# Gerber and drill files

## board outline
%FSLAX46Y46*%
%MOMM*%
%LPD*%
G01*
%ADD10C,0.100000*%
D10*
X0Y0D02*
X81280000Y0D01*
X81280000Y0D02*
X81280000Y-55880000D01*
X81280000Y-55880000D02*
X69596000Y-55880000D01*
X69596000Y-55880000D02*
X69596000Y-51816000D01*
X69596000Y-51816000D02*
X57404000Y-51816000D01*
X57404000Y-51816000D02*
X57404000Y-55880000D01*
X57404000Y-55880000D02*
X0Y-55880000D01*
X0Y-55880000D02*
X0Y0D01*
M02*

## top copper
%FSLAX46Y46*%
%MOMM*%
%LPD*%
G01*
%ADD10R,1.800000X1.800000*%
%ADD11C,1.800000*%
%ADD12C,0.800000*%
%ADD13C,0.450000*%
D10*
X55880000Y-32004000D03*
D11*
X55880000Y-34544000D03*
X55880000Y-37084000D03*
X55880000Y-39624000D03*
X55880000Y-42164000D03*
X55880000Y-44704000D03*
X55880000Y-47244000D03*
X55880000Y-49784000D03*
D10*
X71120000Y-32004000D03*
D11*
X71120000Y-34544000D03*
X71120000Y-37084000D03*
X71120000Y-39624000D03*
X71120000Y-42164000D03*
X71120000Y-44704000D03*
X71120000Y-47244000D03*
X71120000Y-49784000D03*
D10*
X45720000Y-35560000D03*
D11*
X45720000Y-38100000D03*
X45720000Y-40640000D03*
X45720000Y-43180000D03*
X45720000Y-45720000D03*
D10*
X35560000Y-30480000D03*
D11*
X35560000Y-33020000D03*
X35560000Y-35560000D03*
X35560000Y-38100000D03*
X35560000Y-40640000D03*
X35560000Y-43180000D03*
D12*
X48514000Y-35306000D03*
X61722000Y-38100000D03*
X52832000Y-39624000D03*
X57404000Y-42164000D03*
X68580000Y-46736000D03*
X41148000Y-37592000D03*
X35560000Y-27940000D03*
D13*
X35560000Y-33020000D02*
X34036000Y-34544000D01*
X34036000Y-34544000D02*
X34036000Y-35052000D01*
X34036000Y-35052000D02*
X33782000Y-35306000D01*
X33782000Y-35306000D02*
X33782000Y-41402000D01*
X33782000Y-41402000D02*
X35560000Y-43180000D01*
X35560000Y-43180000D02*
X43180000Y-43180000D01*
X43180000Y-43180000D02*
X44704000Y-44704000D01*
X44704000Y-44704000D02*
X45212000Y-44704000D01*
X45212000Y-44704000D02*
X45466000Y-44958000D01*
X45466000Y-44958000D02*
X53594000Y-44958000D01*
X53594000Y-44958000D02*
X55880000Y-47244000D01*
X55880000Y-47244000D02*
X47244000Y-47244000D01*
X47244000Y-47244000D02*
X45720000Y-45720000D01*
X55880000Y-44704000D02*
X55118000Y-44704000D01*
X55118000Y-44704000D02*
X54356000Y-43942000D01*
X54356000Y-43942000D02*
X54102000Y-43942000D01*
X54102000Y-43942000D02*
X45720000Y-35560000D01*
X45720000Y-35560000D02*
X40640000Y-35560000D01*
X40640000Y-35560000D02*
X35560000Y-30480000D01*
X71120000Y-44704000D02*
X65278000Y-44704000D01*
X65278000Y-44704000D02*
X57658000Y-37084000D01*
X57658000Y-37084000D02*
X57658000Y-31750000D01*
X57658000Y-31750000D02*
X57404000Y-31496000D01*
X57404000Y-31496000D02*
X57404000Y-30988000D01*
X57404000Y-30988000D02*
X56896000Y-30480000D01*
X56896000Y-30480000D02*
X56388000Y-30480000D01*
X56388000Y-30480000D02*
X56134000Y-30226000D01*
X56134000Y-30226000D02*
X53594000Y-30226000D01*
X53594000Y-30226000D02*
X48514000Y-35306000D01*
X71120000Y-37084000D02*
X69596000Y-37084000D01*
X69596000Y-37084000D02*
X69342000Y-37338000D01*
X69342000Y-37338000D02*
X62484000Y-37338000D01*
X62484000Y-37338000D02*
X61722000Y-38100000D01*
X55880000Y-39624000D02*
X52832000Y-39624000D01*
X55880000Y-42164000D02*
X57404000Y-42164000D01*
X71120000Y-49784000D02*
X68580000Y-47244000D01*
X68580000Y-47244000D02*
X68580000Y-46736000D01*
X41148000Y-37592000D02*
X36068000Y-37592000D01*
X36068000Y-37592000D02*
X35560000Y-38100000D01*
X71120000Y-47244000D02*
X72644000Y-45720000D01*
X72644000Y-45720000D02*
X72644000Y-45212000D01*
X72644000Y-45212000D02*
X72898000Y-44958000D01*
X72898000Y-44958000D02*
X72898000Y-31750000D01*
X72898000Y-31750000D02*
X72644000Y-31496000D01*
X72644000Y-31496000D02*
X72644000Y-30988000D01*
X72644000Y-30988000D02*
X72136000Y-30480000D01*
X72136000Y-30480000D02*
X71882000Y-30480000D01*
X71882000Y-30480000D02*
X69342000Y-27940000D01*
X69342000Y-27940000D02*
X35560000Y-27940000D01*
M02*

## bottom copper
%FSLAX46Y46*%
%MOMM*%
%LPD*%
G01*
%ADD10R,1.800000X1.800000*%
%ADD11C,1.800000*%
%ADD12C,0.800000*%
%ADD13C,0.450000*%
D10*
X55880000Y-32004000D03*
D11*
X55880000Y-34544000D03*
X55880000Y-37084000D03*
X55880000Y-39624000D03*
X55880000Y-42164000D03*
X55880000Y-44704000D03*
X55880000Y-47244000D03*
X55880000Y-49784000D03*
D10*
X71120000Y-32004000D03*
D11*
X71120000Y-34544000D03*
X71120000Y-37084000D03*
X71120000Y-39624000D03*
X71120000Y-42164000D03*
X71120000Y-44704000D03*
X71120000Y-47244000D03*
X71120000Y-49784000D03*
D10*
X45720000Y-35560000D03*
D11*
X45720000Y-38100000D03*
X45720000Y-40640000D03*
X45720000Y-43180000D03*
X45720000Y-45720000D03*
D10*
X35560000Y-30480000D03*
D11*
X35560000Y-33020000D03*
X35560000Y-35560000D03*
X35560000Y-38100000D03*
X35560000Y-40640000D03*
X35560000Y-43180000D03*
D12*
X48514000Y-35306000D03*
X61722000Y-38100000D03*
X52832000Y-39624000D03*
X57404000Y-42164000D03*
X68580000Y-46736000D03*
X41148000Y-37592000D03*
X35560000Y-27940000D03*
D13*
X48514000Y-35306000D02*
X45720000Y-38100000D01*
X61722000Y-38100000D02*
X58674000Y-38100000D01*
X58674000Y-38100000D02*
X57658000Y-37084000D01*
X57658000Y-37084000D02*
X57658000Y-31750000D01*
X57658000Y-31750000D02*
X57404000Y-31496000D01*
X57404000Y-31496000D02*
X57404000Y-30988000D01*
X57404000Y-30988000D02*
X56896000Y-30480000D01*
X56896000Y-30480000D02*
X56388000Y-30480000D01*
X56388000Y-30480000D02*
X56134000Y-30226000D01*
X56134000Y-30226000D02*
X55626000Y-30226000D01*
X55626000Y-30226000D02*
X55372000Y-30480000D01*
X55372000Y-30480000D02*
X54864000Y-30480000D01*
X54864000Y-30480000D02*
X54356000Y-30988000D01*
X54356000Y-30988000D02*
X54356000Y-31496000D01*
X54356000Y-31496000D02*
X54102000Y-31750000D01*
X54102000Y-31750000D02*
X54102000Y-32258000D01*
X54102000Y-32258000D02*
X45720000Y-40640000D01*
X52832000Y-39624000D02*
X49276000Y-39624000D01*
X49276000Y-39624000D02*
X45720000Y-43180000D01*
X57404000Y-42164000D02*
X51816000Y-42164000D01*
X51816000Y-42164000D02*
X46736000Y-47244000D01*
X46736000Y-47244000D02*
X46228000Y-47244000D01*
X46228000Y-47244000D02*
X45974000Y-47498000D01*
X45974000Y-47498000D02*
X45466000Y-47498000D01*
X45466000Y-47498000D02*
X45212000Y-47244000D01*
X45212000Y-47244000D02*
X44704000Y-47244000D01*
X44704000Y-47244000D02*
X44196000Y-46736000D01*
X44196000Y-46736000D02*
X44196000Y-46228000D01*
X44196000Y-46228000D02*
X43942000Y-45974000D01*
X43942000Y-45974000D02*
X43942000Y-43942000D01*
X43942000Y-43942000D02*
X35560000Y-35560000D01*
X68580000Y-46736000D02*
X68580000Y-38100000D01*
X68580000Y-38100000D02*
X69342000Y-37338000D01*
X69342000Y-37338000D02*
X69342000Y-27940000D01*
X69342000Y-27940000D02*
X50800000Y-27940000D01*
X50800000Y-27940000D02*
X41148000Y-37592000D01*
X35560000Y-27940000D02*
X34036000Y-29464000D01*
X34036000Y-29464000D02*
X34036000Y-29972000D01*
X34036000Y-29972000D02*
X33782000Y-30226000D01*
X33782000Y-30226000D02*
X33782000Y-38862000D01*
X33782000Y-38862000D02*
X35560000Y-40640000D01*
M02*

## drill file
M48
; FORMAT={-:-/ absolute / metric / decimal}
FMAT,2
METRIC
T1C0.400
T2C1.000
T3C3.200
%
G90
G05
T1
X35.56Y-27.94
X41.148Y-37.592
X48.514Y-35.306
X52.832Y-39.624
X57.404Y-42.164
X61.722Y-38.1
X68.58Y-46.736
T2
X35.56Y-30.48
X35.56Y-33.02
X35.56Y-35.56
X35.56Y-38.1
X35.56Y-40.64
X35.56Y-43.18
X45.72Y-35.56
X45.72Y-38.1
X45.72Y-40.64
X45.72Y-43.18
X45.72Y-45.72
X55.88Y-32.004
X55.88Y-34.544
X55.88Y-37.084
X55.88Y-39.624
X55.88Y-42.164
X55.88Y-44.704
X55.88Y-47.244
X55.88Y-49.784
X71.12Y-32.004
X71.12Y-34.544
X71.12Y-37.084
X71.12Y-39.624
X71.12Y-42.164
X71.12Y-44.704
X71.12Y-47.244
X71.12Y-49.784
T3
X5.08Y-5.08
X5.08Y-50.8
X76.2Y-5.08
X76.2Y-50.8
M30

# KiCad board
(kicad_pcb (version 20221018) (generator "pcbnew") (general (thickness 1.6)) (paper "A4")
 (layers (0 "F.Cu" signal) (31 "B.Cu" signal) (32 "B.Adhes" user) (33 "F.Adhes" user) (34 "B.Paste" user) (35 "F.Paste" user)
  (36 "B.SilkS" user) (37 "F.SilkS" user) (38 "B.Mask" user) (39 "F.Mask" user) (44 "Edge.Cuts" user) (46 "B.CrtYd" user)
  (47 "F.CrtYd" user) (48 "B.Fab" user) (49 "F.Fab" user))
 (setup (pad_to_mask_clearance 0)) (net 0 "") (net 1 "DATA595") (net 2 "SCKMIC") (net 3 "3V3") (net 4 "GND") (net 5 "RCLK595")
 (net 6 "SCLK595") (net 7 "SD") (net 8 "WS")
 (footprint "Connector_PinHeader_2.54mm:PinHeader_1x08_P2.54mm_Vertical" (layer "F.Cu") (at 55.8800 32.0040)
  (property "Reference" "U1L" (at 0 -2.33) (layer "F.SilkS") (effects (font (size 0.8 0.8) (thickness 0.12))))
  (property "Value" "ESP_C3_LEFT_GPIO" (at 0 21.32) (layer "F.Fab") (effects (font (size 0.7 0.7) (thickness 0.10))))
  (pad "1" thru_hole rect (at 0 0.0000) (size 1.8 1.8) (drill 1.0) (layers "*.Cu" "*.Mask") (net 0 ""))
  (pad "2" thru_hole circle (at 0 2.5400) (size 1.8 1.8) (drill 1.0) (layers "*.Cu" "*.Mask") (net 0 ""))
  (pad "3" thru_hole circle (at 0 5.0800) (size 1.8 1.8) (drill 1.0) (layers "*.Cu" "*.Mask") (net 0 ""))
  (pad "4" thru_hole circle (at 0 7.6200) (size 1.8 1.8) (drill 1.0) (layers "*.Cu" "*.Mask") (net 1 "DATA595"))
  (pad "5" thru_hole circle (at 0 10.1600) (size 1.8 1.8) (drill 1.0) (layers "*.Cu" "*.Mask") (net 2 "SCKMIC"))
  (pad "6" thru_hole circle (at 0 12.7000) (size 1.8 1.8) (drill 1.0) (layers "*.Cu" "*.Mask") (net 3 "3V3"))
  (pad "7" thru_hole circle (at 0 15.2400) (size 1.8 1.8) (drill 1.0) (layers "*.Cu" "*.Mask") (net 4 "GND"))
  (pad "8" thru_hole circle (at 0 17.7800) (size 1.8 1.8) (drill 1.0) (layers "*.Cu" "*.Mask") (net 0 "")))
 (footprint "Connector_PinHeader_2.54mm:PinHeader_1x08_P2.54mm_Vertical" (layer "F.Cu") (at 71.1200 32.0040)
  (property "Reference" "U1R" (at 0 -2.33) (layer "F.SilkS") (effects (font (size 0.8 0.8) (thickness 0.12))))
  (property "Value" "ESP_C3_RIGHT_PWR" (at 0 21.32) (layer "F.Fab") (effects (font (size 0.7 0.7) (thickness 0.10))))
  (pad "1" thru_hole rect (at 0 0.0000) (size 1.8 1.8) (drill 1.0) (layers "*.Cu" "*.Mask") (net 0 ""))
  (pad "2" thru_hole circle (at 0 2.5400) (size 1.8 1.8) (drill 1.0) (layers "*.Cu" "*.Mask") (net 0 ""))
  (pad "3" thru_hole circle (at 0 5.0800) (size 1.8 1.8) (drill 1.0) (layers "*.Cu" "*.Mask") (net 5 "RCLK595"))
  (pad "4" thru_hole circle (at 0 7.6200) (size 1.8 1.8) (drill 1.0) (layers "*.Cu" "*.Mask") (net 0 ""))
  (pad "5" thru_hole circle (at 0 10.1600) (size 1.8 1.8) (drill 1.0) (layers "*.Cu" "*.Mask") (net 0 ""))
  (pad "6" thru_hole circle (at 0 12.7000) (size 1.8 1.8) (drill 1.0) (layers "*.Cu" "*.Mask") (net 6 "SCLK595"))
  (pad "7" thru_hole circle (at 0 15.2400) (size 1.8 1.8) (drill 1.0) (layers "*.Cu" "*.Mask") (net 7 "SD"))
  (pad "8" thru_hole circle (at 0 17.7800) (size 1.8 1.8) (drill 1.0) (layers "*.Cu" "*.Mask") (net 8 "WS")))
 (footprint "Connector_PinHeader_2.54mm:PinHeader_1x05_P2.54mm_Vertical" (layer "F.Cu") (at 45.7200 35.5600)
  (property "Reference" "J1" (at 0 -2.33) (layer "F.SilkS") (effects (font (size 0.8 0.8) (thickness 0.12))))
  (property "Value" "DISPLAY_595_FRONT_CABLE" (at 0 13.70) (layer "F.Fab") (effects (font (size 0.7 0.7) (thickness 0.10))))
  (pad "1" thru_hole rect (at 0 0.0000) (size 1.8 1.8) (drill 1.0) (layers "*.Cu" "*.Mask") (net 3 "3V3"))
  (pad "2" thru_hole circle (at 0 2.5400) (size 1.8 1.8) (drill 1.0) (layers "*.Cu" "*.Mask") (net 6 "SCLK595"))
  (pad "3" thru_hole circle (at 0 5.0800) (size 1.8 1.8) (drill 1.0) (layers "*.Cu" "*.Mask") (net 5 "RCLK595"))
  (pad "4" thru_hole circle (at 0 7.6200) (size 1.8 1.8) (drill 1.0) (layers "*.Cu" "*.Mask") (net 1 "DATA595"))
  (pad "5" thru_hole circle (at 0 10.1600) (size 1.8 1.8) (drill 1.0) (layers "*.Cu" "*.Mask") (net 4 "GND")))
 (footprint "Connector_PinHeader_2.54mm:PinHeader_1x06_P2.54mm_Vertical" (layer "F.Cu") (at 35.5600 30.4800)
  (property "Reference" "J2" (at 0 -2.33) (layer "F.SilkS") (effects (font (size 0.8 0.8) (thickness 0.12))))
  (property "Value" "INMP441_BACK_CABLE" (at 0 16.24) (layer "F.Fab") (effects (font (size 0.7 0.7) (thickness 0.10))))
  (pad "1" thru_hole rect (at 0 0.0000) (size 1.8 1.8) (drill 1.0) (layers "*.Cu" "*.Mask") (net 3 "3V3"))
  (pad "2" thru_hole circle (at 0 2.5400) (size 1.8 1.8) (drill 1.0) (layers "*.Cu" "*.Mask") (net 4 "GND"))
  (pad "3" thru_hole circle (at 0 5.0800) (size 1.8 1.8) (drill 1.0) (layers "*.Cu" "*.Mask") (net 2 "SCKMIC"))
  (pad "4" thru_hole circle (at 0 7.6200) (size 1.8 1.8) (drill 1.0) (layers "*.Cu" "*.Mask") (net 8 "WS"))
  (pad "5" thru_hole circle (at 0 10.1600) (size 1.8 1.8) (drill 1.0) (layers "*.Cu" "*.Mask") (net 7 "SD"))
  (pad "6" thru_hole circle (at 0 12.7000) (size 1.8 1.8) (drill 1.0) (layers "*.Cu" "*.Mask") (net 4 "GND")))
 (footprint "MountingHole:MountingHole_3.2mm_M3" (layer "F.Cu") (at 5.080 5.080)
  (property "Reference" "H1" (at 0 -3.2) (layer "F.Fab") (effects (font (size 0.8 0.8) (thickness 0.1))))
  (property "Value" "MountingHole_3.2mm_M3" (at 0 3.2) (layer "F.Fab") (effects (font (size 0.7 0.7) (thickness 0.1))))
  (pad "" np_thru_hole circle (at 0 0) (size 3.2 3.2) (drill 3.2) (layers "*.Cu" "*.Mask")))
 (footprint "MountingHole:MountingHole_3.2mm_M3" (layer "F.Cu") (at 76.200 5.080)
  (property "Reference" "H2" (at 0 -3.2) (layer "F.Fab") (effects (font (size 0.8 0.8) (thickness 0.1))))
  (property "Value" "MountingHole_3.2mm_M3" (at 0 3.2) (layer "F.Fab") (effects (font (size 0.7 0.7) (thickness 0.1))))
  (pad "" np_thru_hole circle (at 0 0) (size 3.2 3.2) (drill 3.2) (layers "*.Cu" "*.Mask")))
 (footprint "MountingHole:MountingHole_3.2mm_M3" (layer "F.Cu") (at 5.080 50.800)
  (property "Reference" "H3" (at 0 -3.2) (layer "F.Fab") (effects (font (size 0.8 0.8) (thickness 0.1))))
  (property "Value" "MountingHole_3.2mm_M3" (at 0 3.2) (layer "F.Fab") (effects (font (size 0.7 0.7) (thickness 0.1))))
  (pad "" np_thru_hole circle (at 0 0) (size 3.2 3.2) (drill 3.2) (layers "*.Cu" "*.Mask")))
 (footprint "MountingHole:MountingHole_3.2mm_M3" (layer "F.Cu") (at 76.200 50.800)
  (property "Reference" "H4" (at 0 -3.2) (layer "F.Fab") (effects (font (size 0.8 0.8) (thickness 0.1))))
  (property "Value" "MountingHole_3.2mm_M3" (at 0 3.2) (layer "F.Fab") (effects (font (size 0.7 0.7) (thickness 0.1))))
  (pad "" np_thru_hole circle (at 0 0) (size 3.2 3.2) (drill 3.2) (layers "*.Cu" "*.Mask")))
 (gr_line (start 0.0000 0.0000) (end 81.2800 0.0000) (stroke (width 0.1) (type default)) (layer "Edge.Cuts"))
 (gr_line (start 81.2800 0.0000) (end 81.2800 55.8800) (stroke (width 0.1) (type default)) (layer "Edge.Cuts"))
 (gr_line (start 81.2800 55.8800) (end 69.5960 55.8800) (stroke (width 0.1) (type default)) (layer "Edge.Cuts"))
 (gr_line (start 69.5960 55.8800) (end 69.5960 51.8160) (stroke (width 0.1) (type default)) (layer "Edge.Cuts"))
 (gr_line (start 69.5960 51.8160) (end 57.4040 51.8160) (stroke (width 0.1) (type default)) (layer "Edge.Cuts"))
 (gr_line (start 57.4040 51.8160) (end 57.4040 55.8800) (stroke (width 0.1) (type default)) (layer "Edge.Cuts"))
 (gr_line (start 57.4040 55.8800) (end 0.0000 55.8800) (stroke (width 0.1) (type default)) (layer "Edge.Cuts"))
 (gr_line (start 0.0000 55.8800) (end 0.0000 0.0000) (stroke (width 0.1) (type default)) (layer "Edge.Cuts"))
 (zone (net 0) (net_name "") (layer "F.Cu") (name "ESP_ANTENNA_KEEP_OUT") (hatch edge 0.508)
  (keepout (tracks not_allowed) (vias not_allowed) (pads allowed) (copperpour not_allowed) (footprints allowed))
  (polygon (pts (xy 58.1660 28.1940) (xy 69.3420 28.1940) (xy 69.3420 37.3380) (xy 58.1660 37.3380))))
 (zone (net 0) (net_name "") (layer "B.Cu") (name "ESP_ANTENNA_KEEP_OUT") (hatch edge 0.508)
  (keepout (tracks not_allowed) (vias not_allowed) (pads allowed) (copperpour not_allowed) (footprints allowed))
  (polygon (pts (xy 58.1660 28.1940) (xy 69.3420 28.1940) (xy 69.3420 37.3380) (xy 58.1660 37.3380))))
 (segment (start 35.5600 33.0200) (end 34.0360 34.5440) (width 0.45) (layer "F.Cu") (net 4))
 (segment (start 34.0360 34.5440) (end 34.0360 35.0520) (width 0.45) (layer "F.Cu") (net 4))
 (segment (start 34.0360 35.0520) (end 33.7820 35.3060) (width 0.45) (layer "F.Cu") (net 4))
 (segment (start 33.7820 35.3060) (end 33.7820 41.4020) (width 0.45) (layer "F.Cu") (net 4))
 (segment (start 33.7820 41.4020) (end 35.5600 43.1800) (width 0.45) (layer "F.Cu") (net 4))
 (segment (start 35.5600 43.1800) (end 43.1800 43.1800) (width 0.45) (layer "F.Cu") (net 4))
 (segment (start 43.1800 43.1800) (end 44.7040 44.7040) (width 0.45) (layer "F.Cu") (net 4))
 (segment (start 44.7040 44.7040) (end 45.2120 44.7040) (width 0.45) (layer "F.Cu") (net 4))
 (segment (start 45.2120 44.7040) (end 45.4660 44.9580) (width 0.45) (layer "F.Cu") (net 4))
 (segment (start 45.4660 44.9580) (end 53.5940 44.9580) (width 0.45) (layer "F.Cu") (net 4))
 (segment (start 53.5940 44.9580) (end 55.8800 47.2440) (width 0.45) (layer "F.Cu") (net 4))
 (segment (start 55.8800 47.2440) (end 47.2440 47.2440) (width 0.45) (layer "F.Cu") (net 4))
 (segment (start 47.2440 47.2440) (end 45.7200 45.7200) (width 0.45) (layer "F.Cu") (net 4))
 (segment (start 55.8800 44.7040) (end 55.1180 44.7040) (width 0.45) (layer "F.Cu") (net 3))
 (segment (start 55.1180 44.7040) (end 54.3560 43.9420) (width 0.45) (layer "F.Cu") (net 3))
 (segment (start 54.3560 43.9420) (end 54.1020 43.9420) (width 0.45) (layer "F.Cu") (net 3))
 (segment (start 54.1020 43.9420) (end 45.7200 35.5600) (width 0.45) (layer "F.Cu") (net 3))
 (segment (start 45.7200 35.5600) (end 40.6400 35.5600) (width 0.45) (layer "F.Cu") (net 3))
 (segment (start 40.6400 35.5600) (end 35.5600 30.4800) (width 0.45) (layer "F.Cu") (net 3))
 (segment (start 71.1200 44.7040) (end 65.2780 44.7040) (width 0.45) (layer "F.Cu") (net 6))
 (segment (start 65.2780 44.7040) (end 57.6580 37.0840) (width 0.45) (layer "F.Cu") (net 6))
 (segment (start 57.6580 37.0840) (end 57.6580 31.7500) (width 0.45) (layer "F.Cu") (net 6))
 (segment (start 57.6580 31.7500) (end 57.4040 31.4960) (width 0.45) (layer "F.Cu") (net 6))
 (segment (start 57.4040 31.4960) (end 57.4040 30.9880) (width 0.45) (layer "F.Cu") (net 6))
 (segment (start 57.4040 30.9880) (end 56.8960 30.4800) (width 0.45) (layer "F.Cu") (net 6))
 (segment (start 56.8960 30.4800) (end 56.3880 30.4800) (width 0.45) (layer "F.Cu") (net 6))
 (segment (start 56.3880 30.4800) (end 56.1340 30.2260) (width 0.45) (layer "F.Cu") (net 6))
 (segment (start 56.1340 30.2260) (end 53.5940 30.2260) (width 0.45) (layer "F.Cu") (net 6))
 (segment (start 53.5940 30.2260) (end 48.5140 35.3060) (width 0.45) (layer "F.Cu") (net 6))
 (segment (start 48.5140 35.3060) (end 45.7200 38.1000) (width 0.45) (layer "B.Cu") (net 6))
 (segment (start 71.1200 37.0840) (end 69.5960 37.0840) (width 0.45) (layer "F.Cu") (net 5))
 (segment (start 69.5960 37.0840) (end 69.3420 37.3380) (width 0.45) (layer "F.Cu") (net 5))
 (segment (start 69.3420 37.3380) (end 62.4840 37.3380) (width 0.45) (layer "F.Cu") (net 5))
 (segment (start 62.4840 37.3380) (end 61.7220 38.1000) (width 0.45) (layer "F.Cu") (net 5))
 (segment (start 61.7220 38.1000) (end 58.6740 38.1000) (width 0.45) (layer "B.Cu") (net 5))
 (segment (start 58.6740 38.1000) (end 57.6580 37.0840) (width 0.45) (layer "B.Cu") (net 5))
 (segment (start 57.6580 37.0840) (end 57.6580 31.7500) (width 0.45) (layer "B.Cu") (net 5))
 (segment (start 57.6580 31.7500) (end 57.4040 31.4960) (width 0.45) (layer "B.Cu") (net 5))
 (segment (start 57.4040 31.4960) (end 57.4040 30.9880) (width 0.45) (layer "B.Cu") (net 5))
 (segment (start 57.4040 30.9880) (end 56.8960 30.4800) (width 0.45) (layer "B.Cu") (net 5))
 (segment (start 56.8960 30.4800) (end 56.3880 30.4800) (width 0.45) (layer "B.Cu") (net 5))
 (segment (start 56.3880 30.4800) (end 56.1340 30.2260) (width 0.45) (layer "B.Cu") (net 5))
 (segment (start 56.1340 30.2260) (end 55.6260 30.2260) (width 0.45) (layer "B.Cu") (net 5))
 (segment (start 55.6260 30.2260) (end 55.3720 30.4800) (width 0.45) (layer "B.Cu") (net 5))
 (segment (start 55.3720 30.4800) (end 54.8640 30.4800) (width 0.45) (layer "B.Cu") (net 5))
 (segment (start 54.8640 30.4800) (end 54.3560 30.9880) (width 0.45) (layer "B.Cu") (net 5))
 (segment (start 54.3560 30.9880) (end 54.3560 31.4960) (width 0.45) (layer "B.Cu") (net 5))
 (segment (start 54.3560 31.4960) (end 54.1020 31.7500) (width 0.45) (layer "B.Cu") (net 5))
 (segment (start 54.1020 31.7500) (end 54.1020 32.2580) (width 0.45) (layer "B.Cu") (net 5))
 (segment (start 54.1020 32.2580) (end 45.7200 40.6400) (width 0.45) (layer "B.Cu") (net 5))
 (segment (start 55.8800 39.6240) (end 52.8320 39.6240) (width 0.45) (layer "F.Cu") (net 1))
 (segment (start 52.8320 39.6240) (end 49.2760 39.6240) (width 0.45) (layer "B.Cu") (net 1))
 (segment (start 49.2760 39.6240) (end 45.7200 43.1800) (width 0.45) (layer "B.Cu") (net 1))
 (segment (start 55.8800 42.1640) (end 57.4040 42.1640) (width 0.45) (layer "F.Cu") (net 2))
 (segment (start 57.4040 42.1640) (end 51.8160 42.1640) (width 0.45) (layer "B.Cu") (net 2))
 (segment (start 51.8160 42.1640) (end 46.7360 47.2440) (width 0.45) (layer "B.Cu") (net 2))
 (segment (start 46.7360 47.2440) (end 46.2280 47.2440) (width 0.45) (layer "B.Cu") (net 2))
 (segment (start 46.2280 47.2440) (end 45.9740 47.4980) (width 0.45) (layer "B.Cu") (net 2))
 (segment (start 45.9740 47.4980) (end 45.4660 47.4980) (width 0.45) (layer "B.Cu") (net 2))
 (segment (start 45.4660 47.4980) (end 45.2120 47.2440) (width 0.45) (layer "B.Cu") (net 2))
 (segment (start 45.2120 47.2440) (end 44.7040 47.2440) (width 0.45) (layer "B.Cu") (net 2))
 (segment (start 44.7040 47.2440) (end 44.1960 46.7360) (width 0.45) (layer "B.Cu") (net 2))
 (segment (start 44.1960 46.7360) (end 44.1960 46.2280) (width 0.45) (layer "B.Cu") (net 2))
 (segment (start 44.1960 46.2280) (end 43.9420 45.9740) (width 0.45) (layer "B.Cu") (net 2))
 (segment (start 43.9420 45.9740) (end 43.9420 43.9420) (width 0.45) (layer "B.Cu") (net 2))
 (segment (start 43.9420 43.9420) (end 35.5600 35.5600) (width 0.45) (layer "B.Cu") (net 2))
 (segment (start 71.1200 49.7840) (end 68.5800 47.2440) (width 0.45) (layer "F.Cu") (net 8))
 (segment (start 68.5800 47.2440) (end 68.5800 46.7360) (width 0.45) (layer "F.Cu") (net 8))
 (segment (start 68.5800 46.7360) (end 68.5800 38.1000) (width 0.45) (layer "B.Cu") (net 8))
 (segment (start 68.5800 38.1000) (end 69.3420 37.3380) (width 0.45) (layer "B.Cu") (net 8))
 (segment (start 69.3420 37.3380) (end 69.3420 27.9400) (width 0.45) (layer "B.Cu") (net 8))
 (segment (start 69.3420 27.9400) (end 50.8000 27.9400) (width 0.45) (layer "B.Cu") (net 8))
 (segment (start 50.8000 27.9400) (end 41.1480 37.5920) (width 0.45) (layer "B.Cu") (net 8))
 (segment (start 41.1480 37.5920) (end 36.0680 37.5920) (width 0.45) (layer "F.Cu") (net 8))
 (segment (start 36.0680 37.5920) (end 35.5600 38.1000) (width 0.45) (layer "F.Cu") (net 8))
 (segment (start 71.1200 47.2440) (end 72.6440 45.7200) (width 0.45) (layer "F.Cu") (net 7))
 (segment (start 72.6440 45.7200) (end 72.6440 45.2120) (width 0.45) (layer "F.Cu") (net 7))
 (segment (start 72.6440 45.2120) (end 72.8980 44.9580) (width 0.45) (layer "F.Cu") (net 7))
 (segment (start 72.8980 44.9580) (end 72.8980 31.7500) (width 0.45) (layer "F.Cu") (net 7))
 (segment (start 72.8980 31.7500) (end 72.6440 31.4960) (width 0.45) (layer "F.Cu") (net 7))
 (segment (start 72.6440 31.4960) (end 72.6440 30.9880) (width 0.45) (layer "F.Cu") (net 7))
 (segment (start 72.6440 30.9880) (end 72.1360 30.4800) (width 0.45) (layer "F.Cu") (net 7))
 (segment (start 72.1360 30.4800) (end 71.8820 30.4800) (width 0.45) (layer "F.Cu") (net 7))
 (segment (start 71.8820 30.4800) (end 69.3420 27.9400) (width 0.45) (layer "F.Cu") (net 7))
 (segment (start 69.3420 27.9400) (end 35.5600 27.9400) (width 0.45) (layer "F.Cu") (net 7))
 (segment (start 35.5600 27.9400) (end 34.0360 29.4640) (width 0.45) (layer "B.Cu") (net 7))
 (segment (start 34.0360 29.4640) (end 34.0360 29.9720) (width 0.45) (layer "B.Cu") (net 7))
 (segment (start 34.0360 29.9720) (end 33.7820 30.2260) (width 0.45) (layer "B.Cu") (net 7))
 (segment (start 33.7820 30.2260) (end 33.7820 38.8620) (width 0.45) (layer "B.Cu") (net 7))
 (segment (start 33.7820 38.8620) (end 35.5600 40.6400) (width 0.45) (layer "B.Cu") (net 7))
 (via (at 48.5140 35.3060) (size 0.8) (drill 0.4) (layers "F.Cu" "B.Cu") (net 6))
 (via (at 61.7220 38.1000) (size 0.8) (drill 0.4) (layers "F.Cu" "B.Cu") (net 5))
 (via (at 52.8320 39.6240) (size 0.8) (drill 0.4) (layers "F.Cu" "B.Cu") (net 1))
 (via (at 57.4040 42.1640) (size 0.8) (drill 0.4) (layers "F.Cu" "B.Cu") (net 2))
 (via (at 68.5800 46.7360) (size 0.8) (drill 0.4) (layers "F.Cu" "B.Cu") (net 8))
 (via (at 41.1480 37.5920) (size 0.8) (drill 0.4) (layers "F.Cu" "B.Cu") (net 8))
 (via (at 35.5600 27.9400) (size 0.8) (drill 0.4) (layers "F.Cu" "B.Cu") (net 7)))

